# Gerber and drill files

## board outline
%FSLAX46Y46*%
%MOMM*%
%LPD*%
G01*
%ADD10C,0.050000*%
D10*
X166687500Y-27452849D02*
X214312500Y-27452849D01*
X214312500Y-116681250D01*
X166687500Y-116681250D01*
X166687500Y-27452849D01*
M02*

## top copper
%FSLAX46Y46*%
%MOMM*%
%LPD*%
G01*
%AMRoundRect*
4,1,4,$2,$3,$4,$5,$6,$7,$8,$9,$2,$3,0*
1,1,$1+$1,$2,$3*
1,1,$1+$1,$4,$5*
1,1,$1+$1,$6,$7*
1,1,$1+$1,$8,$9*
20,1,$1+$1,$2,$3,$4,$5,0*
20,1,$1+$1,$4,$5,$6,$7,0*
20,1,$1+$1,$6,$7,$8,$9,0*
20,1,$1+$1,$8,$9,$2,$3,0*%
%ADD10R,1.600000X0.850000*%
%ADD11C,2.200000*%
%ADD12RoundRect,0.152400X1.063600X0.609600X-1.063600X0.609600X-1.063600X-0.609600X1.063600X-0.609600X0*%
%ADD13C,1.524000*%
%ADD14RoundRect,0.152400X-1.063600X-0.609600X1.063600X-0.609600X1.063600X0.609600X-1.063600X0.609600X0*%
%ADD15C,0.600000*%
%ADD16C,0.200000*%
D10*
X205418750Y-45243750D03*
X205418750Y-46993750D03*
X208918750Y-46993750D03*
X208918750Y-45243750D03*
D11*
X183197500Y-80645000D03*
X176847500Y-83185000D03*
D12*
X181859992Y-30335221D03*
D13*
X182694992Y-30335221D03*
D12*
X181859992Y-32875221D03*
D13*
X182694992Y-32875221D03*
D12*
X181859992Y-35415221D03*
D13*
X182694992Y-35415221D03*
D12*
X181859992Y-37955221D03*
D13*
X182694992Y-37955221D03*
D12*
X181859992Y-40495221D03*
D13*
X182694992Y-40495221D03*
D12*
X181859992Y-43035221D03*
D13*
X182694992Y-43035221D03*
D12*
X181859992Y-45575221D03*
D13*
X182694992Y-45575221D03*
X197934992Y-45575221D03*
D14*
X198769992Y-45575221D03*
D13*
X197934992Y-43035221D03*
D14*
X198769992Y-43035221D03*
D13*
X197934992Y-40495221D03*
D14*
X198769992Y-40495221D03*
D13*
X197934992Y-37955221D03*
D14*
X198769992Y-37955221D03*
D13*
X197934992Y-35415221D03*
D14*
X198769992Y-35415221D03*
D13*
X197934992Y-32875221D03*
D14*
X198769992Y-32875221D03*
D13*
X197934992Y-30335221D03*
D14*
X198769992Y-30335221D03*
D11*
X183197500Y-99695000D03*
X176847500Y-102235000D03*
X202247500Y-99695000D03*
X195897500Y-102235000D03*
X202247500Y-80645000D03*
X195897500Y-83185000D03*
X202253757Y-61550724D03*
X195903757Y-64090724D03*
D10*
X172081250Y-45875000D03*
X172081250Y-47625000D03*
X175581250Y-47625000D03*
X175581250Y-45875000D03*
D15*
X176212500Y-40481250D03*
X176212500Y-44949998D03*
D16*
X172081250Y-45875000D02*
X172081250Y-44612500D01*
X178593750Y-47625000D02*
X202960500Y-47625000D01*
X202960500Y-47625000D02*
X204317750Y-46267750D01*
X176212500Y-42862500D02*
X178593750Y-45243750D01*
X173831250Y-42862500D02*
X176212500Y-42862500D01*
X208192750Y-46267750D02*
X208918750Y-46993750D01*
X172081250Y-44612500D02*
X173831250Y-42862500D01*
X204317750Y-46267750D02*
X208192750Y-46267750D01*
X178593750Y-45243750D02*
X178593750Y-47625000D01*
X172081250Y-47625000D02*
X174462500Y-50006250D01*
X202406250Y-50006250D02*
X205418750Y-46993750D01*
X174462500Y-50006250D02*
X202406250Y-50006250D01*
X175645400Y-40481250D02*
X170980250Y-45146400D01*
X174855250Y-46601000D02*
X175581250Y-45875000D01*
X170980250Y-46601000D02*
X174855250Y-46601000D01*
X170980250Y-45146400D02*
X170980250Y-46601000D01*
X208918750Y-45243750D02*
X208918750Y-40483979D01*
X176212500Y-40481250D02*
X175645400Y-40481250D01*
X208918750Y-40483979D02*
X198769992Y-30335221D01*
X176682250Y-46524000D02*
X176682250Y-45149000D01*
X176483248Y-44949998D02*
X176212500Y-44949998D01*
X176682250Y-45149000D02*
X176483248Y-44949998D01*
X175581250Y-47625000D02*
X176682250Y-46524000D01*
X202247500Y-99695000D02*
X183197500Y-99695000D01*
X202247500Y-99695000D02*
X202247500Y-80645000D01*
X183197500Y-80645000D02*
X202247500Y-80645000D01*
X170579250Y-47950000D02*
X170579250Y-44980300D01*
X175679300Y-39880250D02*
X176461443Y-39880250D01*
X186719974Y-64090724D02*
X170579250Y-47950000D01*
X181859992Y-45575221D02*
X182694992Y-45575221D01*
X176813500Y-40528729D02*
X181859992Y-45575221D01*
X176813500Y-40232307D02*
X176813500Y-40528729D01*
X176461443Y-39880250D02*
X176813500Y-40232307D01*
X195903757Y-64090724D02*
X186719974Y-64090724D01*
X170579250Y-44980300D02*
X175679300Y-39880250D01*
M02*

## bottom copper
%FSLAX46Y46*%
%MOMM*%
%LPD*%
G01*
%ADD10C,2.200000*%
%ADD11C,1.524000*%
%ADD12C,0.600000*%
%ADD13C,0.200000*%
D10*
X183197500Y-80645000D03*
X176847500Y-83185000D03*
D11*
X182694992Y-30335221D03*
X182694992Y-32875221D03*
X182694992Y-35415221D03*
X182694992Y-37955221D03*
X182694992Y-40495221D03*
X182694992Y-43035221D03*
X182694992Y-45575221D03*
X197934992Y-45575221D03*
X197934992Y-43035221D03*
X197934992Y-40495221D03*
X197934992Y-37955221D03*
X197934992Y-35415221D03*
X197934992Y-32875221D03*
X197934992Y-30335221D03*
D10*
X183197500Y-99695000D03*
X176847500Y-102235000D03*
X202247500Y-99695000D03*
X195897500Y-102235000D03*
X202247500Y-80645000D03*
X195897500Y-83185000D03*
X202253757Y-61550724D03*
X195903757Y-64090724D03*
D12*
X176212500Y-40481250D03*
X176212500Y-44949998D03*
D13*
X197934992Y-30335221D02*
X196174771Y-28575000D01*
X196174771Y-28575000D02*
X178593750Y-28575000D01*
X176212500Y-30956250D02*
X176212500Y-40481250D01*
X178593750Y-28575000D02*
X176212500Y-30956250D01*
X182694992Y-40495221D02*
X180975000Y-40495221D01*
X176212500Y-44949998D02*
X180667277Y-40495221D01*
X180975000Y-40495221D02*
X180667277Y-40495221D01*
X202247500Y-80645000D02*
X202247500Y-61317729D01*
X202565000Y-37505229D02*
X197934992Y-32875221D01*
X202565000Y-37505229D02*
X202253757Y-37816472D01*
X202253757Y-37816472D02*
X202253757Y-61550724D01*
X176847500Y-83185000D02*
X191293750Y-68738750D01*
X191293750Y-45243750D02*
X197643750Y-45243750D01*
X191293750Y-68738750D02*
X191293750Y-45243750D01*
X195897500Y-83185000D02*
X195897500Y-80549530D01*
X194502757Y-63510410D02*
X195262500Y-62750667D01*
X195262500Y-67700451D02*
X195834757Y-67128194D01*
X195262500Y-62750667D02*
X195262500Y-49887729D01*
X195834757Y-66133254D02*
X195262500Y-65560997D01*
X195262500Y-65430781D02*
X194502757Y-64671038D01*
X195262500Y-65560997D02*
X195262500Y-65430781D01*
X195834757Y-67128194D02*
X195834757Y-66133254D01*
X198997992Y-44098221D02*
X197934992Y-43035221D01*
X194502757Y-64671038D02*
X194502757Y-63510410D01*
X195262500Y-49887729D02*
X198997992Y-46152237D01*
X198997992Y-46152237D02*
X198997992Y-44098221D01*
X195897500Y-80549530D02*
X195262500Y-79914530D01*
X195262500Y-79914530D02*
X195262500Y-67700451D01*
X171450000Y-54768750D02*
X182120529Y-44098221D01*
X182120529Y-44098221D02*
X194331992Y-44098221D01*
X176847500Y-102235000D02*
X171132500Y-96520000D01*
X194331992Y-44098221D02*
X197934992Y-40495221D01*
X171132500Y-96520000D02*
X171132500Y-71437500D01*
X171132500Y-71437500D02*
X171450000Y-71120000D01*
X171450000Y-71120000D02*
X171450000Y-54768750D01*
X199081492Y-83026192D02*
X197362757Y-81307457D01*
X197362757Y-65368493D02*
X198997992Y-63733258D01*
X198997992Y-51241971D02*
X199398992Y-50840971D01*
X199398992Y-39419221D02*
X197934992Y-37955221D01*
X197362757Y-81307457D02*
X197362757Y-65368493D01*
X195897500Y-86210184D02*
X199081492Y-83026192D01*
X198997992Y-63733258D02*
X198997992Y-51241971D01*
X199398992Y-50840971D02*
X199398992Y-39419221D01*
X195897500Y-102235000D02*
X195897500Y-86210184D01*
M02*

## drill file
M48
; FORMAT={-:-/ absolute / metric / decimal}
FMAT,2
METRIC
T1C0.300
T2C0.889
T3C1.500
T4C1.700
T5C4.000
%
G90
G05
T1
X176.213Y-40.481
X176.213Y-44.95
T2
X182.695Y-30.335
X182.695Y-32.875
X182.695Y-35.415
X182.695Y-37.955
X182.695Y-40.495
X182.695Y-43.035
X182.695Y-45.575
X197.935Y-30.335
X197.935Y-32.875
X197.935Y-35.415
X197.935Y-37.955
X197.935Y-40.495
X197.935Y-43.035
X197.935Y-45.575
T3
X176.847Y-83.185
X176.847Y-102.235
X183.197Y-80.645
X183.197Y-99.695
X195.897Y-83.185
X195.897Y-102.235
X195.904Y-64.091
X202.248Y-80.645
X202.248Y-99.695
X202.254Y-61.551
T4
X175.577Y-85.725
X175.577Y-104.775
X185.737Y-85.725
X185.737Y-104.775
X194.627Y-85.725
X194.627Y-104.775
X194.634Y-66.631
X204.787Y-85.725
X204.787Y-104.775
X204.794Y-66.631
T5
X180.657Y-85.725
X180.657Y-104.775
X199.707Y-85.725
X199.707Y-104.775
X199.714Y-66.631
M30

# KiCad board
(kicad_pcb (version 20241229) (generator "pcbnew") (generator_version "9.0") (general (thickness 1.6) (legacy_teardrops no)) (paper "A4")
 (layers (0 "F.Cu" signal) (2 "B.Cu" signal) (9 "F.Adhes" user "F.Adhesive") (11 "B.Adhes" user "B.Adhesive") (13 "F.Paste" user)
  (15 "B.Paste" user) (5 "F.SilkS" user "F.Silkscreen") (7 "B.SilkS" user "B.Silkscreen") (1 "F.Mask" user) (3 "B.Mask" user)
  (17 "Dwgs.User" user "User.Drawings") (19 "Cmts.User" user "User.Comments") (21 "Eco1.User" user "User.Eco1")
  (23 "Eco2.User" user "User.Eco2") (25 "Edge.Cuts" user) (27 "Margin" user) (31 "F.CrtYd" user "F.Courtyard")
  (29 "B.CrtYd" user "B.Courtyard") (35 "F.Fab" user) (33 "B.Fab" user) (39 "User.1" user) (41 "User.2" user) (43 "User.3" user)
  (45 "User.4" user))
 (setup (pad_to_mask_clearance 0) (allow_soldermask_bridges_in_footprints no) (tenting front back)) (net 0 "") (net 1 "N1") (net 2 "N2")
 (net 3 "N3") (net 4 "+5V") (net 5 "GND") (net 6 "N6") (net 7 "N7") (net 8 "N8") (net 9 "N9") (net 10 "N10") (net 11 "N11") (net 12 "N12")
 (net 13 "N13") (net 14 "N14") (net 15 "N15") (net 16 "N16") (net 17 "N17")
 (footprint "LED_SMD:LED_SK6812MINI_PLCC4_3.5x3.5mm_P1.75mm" (layer "F.Cu") (at 207.16875 46.11875)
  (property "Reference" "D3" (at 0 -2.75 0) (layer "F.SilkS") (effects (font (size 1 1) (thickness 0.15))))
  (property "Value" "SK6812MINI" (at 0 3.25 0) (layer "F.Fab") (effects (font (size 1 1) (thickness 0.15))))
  (pad "1" smd rect (at -1.75 -0.875) (size 1.6 0.85) (layers "F.Cu" "F.Mask" "F.Paste") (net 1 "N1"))
  (pad "2" smd rect (at -1.75 0.875) (size 1.6 0.85) (layers "F.Cu" "F.Mask" "F.Paste") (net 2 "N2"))
  (pad "3" smd rect (at 1.75 0.875) (size 1.6 0.85) (layers "F.Cu" "F.Mask" "F.Paste") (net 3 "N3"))
  (pad "4" smd rect (at 1.75 -0.875) (size 1.6 0.85) (layers "F.Cu" "F.Mask" "F.Paste") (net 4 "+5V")))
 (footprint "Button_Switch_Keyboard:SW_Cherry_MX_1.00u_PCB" (layer "F.Cu") (at 183.1975 80.645)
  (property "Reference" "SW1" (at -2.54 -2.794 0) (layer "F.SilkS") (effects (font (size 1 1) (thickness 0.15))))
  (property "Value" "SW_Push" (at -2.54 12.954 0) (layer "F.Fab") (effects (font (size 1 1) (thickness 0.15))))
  (pad "" np_thru_hole circle (at -7.62 5.08) (size 1.7 1.7) (drill 1.7) (layers "*.Cu" "*.Mask"))
  (pad "" np_thru_hole circle (at -2.54 5.08) (size 4 4) (drill 4) (layers "*.Cu" "*.Mask"))
  (pad "" np_thru_hole circle (at 2.54 5.08) (size 1.7 1.7) (drill 1.7) (layers "*.Cu" "*.Mask"))
  (pad "1" thru_hole circle (at 0 0) (size 2.2 2.2) (drill 1.5) (layers "*.Cu" "*.Mask") (remove_unused_layers no) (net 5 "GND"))
  (pad "2" thru_hole circle (at -6.35 2.54) (size 2.2 2.2) (drill 1.5) (layers "*.Cu" "*.Mask") (remove_unused_layers no) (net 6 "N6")))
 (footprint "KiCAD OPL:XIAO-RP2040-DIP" (layer "F.Cu") (at 190.314992 37.955221)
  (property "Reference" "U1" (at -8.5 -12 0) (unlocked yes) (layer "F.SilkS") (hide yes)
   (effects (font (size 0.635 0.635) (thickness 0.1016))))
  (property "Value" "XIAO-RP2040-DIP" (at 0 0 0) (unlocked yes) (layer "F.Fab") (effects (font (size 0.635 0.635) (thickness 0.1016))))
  (pad "1" smd roundrect (at -8.455 -7.62 180) (size 2.432 1.524) (layers "F.Cu" "F.Mask") (roundrect_rratio 0.1) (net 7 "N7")
   (thermal_bridge_angle 45))
  (pad "1" thru_hole circle (at -7.62 -7.62 180) (size 1.524 1.524) (drill 0.889) (layers "*.Cu" "*.Mask") (remove_unused_layers no)
   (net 7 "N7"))
  (pad "2" smd roundrect (at -8.455 -5.08 180) (size 2.432 1.524) (layers "F.Cu" "F.Mask") (roundrect_rratio 0.1) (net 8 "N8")
   (thermal_bridge_angle 45))
  (pad "2" thru_hole circle (at -7.62 -5.08 180) (size 1.524 1.524) (drill 0.889) (layers "*.Cu" "*.Mask") (remove_unused_layers no)
   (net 8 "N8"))
  (pad "3" smd roundrect (at -8.455 -2.54 180) (size 2.432 1.524) (layers "F.Cu" "F.Mask") (roundrect_rratio 0.1) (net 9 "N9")
   (thermal_bridge_angle 45))
  (pad "3" thru_hole circle (at -7.62 -2.54 180) (size 1.524 1.524) (drill 0.889) (layers "*.Cu" "*.Mask") (remove_unused_layers no)
   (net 9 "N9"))
  (pad "4" smd roundrect (at -8.455 0 180) (size 2.432 1.524) (layers "F.Cu" "F.Mask") (roundrect_rratio 0.1) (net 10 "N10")
   (thermal_bridge_angle 45))
  (pad "4" thru_hole circle (at -7.62 0 180) (size 1.524 1.524) (drill 0.889) (layers "*.Cu" "*.Mask") (remove_unused_layers no)
   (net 10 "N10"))
  (pad "5" smd roundrect (at -8.455 2.54 180) (size 2.432 1.524) (layers "F.Cu" "F.Mask") (roundrect_rratio 0.1) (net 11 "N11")
   (thermal_bridge_angle 45))
  (pad "5" thru_hole circle (at -7.62 2.54 180) (size 1.524 1.524) (drill 0.889) (layers "*.Cu" "*.Mask") (remove_unused_layers no)
   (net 11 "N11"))
  (pad "6" smd roundrect (at -8.455 5.08 180) (size 2.432 1.524) (layers "F.Cu" "F.Mask") (roundrect_rratio 0.1) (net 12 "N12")
   (thermal_bridge_angle 45))
  (pad "6" thru_hole circle (at -7.62 5.08 180) (size 1.524 1.524) (drill 0.889) (layers "*.Cu" "*.Mask") (remove_unused_layers no)
   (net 12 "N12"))
  (pad "7" smd roundrect (at -8.455 7.62 180) (size 2.432 1.524) (layers "F.Cu" "F.Mask") (roundrect_rratio 0.1) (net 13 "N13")
   (thermal_bridge_angle 45))
  (pad "7" thru_hole circle (at -7.62 7.62 180) (size 1.524 1.524) (drill 0.889) (layers "*.Cu" "*.Mask") (remove_unused_layers no)
   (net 13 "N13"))
  (pad "8" thru_hole circle (at 7.62 7.62) (size 1.524 1.524) (drill 0.889) (layers "*.Cu" "*.Mask") (remove_unused_layers no) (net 6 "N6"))
  (pad "8" smd roundrect (at 8.455 7.62) (size 2.432 1.524) (layers "F.Cu" "F.Mask") (roundrect_rratio 0.1) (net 6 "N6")
   (thermal_bridge_angle 45))
  (pad "9" thru_hole circle (at 7.62 5.08) (size 1.524 1.524) (drill 0.889) (layers "*.Cu" "*.Mask") (remove_unused_layers no)
   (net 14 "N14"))
  (pad "9" smd roundrect (at 8.455 5.08) (size 2.432 1.524) (layers "F.Cu" "F.Mask") (roundrect_rratio 0.1) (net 14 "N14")
   (thermal_bridge_angle 45))
  (pad "10" thru_hole circle (at 7.62 2.54) (size 1.524 1.524) (drill 0.889) (layers "*.Cu" "*.Mask") (remove_unused_layers no)
   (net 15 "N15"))
  (pad "10" smd roundrect (at 8.455 2.54) (size 2.432 1.524) (layers "F.Cu" "F.Mask") (roundrect_rratio 0.1) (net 15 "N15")
   (thermal_bridge_angle 45))
  (pad "11" thru_hole circle (at 7.62 0) (size 1.524 1.524) (drill 0.889) (layers "*.Cu" "*.Mask") (remove_unused_layers no) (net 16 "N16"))
  (pad "11" smd roundrect (at 8.455 0) (size 2.432 1.524) (layers "F.Cu" "F.Mask") (roundrect_rratio 0.1) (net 16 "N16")
   (thermal_bridge_angle 45))
  (pad "12" thru_hole circle (at 7.62 -2.54) (size 1.524 1.524) (drill 0.889) (layers "*.Cu" "*.Mask") (remove_unused_layers no)
   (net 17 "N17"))
  (pad "12" smd roundrect (at 8.455 -2.54) (size 2.432 1.524) (layers "F.Cu" "F.Mask") (roundrect_rratio 0.1) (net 17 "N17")
   (thermal_bridge_angle 45))
  (pad "13" thru_hole circle (at 7.62 -5.08) (size 1.524 1.524) (drill 0.889) (layers "*.Cu" "*.Mask") (remove_unused_layers no)
   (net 5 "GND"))
  (pad "13" smd roundrect (at 8.455 -5.08) (size 2.432 1.524) (layers "F.Cu" "F.Mask") (roundrect_rratio 0.1) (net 5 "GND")
   (thermal_bridge_angle 45))
  (pad "14" thru_hole circle (at 7.62 -7.62) (size 1.524 1.524) (drill 0.889) (layers "*.Cu" "*.Mask") (remove_unused_layers no)
   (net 4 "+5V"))
  (pad "14" smd roundrect (at 8.455 -7.62) (size 2.432 1.524) (layers "F.Cu" "F.Mask") (roundrect_rratio 0.1) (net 4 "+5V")
   (thermal_bridge_angle 45)))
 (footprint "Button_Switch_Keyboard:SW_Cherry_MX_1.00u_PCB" (layer "F.Cu") (at 183.1975 99.695)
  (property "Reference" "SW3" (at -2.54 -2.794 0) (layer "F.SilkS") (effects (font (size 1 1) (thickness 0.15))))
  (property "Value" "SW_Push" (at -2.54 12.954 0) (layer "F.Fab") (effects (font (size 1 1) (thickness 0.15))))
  (pad "" np_thru_hole circle (at -7.62 5.08) (size 1.7 1.7) (drill 1.7) (layers "*.Cu" "*.Mask"))
  (pad "" np_thru_hole circle (at -2.54 5.08) (size 4 4) (drill 4) (layers "*.Cu" "*.Mask"))
  (pad "" np_thru_hole circle (at 2.54 5.08) (size 1.7 1.7) (drill 1.7) (layers "*.Cu" "*.Mask"))
  (pad "1" thru_hole circle (at 0 0) (size 2.2 2.2) (drill 1.5) (layers "*.Cu" "*.Mask") (remove_unused_layers no) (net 5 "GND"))
  (pad "2" thru_hole circle (at -6.35 2.54) (size 2.2 2.2) (drill 1.5) (layers "*.Cu" "*.Mask") (remove_unused_layers no) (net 15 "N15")))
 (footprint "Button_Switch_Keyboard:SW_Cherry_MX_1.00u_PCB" (layer "F.Cu") (at 202.2475 99.695)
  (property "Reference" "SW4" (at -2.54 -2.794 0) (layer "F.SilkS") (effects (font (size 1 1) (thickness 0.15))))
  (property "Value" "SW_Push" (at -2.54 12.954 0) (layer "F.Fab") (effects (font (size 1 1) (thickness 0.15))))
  (pad "" np_thru_hole circle (at -7.62 5.08) (size 1.7 1.7) (drill 1.7) (layers "*.Cu" "*.Mask"))
  (pad "" np_thru_hole circle (at -2.54 5.08) (size 4 4) (drill 4) (layers "*.Cu" "*.Mask"))
  (pad "" np_thru_hole circle (at 2.54 5.08) (size 1.7 1.7) (drill 1.7) (layers "*.Cu" "*.Mask"))
  (pad "1" thru_hole circle (at 0 0) (size 2.2 2.2) (drill 1.5) (layers "*.Cu" "*.Mask") (remove_unused_layers no) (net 5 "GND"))
  (pad "2" thru_hole circle (at -6.35 2.54) (size 2.2 2.2) (drill 1.5) (layers "*.Cu" "*.Mask") (remove_unused_layers no) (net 16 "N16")))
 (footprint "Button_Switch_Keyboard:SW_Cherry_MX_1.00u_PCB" (layer "F.Cu") (at 202.2475 80.645)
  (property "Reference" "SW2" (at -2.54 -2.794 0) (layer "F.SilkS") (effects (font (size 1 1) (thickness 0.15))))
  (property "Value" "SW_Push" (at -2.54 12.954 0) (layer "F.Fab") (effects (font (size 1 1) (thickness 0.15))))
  (pad "" np_thru_hole circle (at -7.62 5.08) (size 1.7 1.7) (drill 1.7) (layers "*.Cu" "*.Mask"))
  (pad "" np_thru_hole circle (at -2.54 5.08) (size 4 4) (drill 4) (layers "*.Cu" "*.Mask"))
  (pad "" np_thru_hole circle (at 2.54 5.08) (size 1.7 1.7) (drill 1.7) (layers "*.Cu" "*.Mask"))
  (pad "1" thru_hole circle (at 0 0) (size 2.2 2.2) (drill 1.5) (layers "*.Cu" "*.Mask") (remove_unused_layers no) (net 5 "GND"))
  (pad "2" thru_hole circle (at -6.35 2.54) (size 2.2 2.2) (drill 1.5) (layers "*.Cu" "*.Mask") (remove_unused_layers no) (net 14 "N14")))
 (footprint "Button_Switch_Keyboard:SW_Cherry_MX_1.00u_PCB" (layer "F.Cu") (at 202.253757 61.550724)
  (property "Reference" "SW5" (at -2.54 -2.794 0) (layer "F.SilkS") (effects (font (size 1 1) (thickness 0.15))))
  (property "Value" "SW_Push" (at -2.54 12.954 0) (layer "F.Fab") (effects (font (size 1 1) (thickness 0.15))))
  (pad "" np_thru_hole circle (at -7.62 5.08) (size 1.7 1.7) (drill 1.7) (layers "*.Cu" "*.Mask"))
  (pad "" np_thru_hole circle (at -2.54 5.08) (size 4 4) (drill 4) (layers "*.Cu" "*.Mask"))
  (pad "" np_thru_hole circle (at 2.54 5.08) (size 1.7 1.7) (drill 1.7) (layers "*.Cu" "*.Mask"))
  (pad "1" thru_hole circle (at 0 0) (size 2.2 2.2) (drill 1.5) (layers "*.Cu" "*.Mask") (remove_unused_layers no) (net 5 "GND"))
  (pad "2" thru_hole circle (at -6.35 2.54) (size 2.2 2.2) (drill 1.5) (layers "*.Cu" "*.Mask") (remove_unused_layers no) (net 13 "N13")))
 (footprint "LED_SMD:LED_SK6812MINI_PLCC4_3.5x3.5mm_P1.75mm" (layer "F.Cu") (at 173.83125 46.75)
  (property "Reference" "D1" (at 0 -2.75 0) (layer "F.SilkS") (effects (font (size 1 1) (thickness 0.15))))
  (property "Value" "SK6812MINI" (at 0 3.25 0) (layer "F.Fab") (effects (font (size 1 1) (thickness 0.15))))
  (pad "1" smd rect (at -1.75 -0.875) (size 1.6 0.85) (layers "F.Cu" "F.Mask" "F.Paste") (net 3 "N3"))
  (pad "2" smd rect (at -1.75 0.875) (size 1.6 0.85) (layers "F.Cu" "F.Mask" "F.Paste") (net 2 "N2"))
  (pad "3" smd rect (at 1.75 0.875) (size 1.6 0.85) (layers "F.Cu" "F.Mask" "F.Paste") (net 11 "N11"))
  (pad "4" smd rect (at 1.75 -0.875) (size 1.6 0.85) (layers "F.Cu" "F.Mask" "F.Paste") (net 4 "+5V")))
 (gr_rect (start 166.6875 27.452849) (end 214.3125 116.68125) (stroke (width 0.05) (type default)) (fill no) (layer "Edge.Cuts"))
 (segment (start 172.08125 45.875) (end 172.08125 44.6125) (width 0.2) (layer "F.Cu") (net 3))
 (segment (start 178.59375 47.625) (end 202.9605 47.625) (width 0.2) (layer "F.Cu") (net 3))
 (segment (start 202.9605 47.625) (end 204.31775 46.26775) (width 0.2) (layer "F.Cu") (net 3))
 (segment (start 176.2125 42.8625) (end 178.59375 45.24375) (width 0.2) (layer "F.Cu") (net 3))
 (segment (start 173.83125 42.8625) (end 176.2125 42.8625) (width 0.2) (layer "F.Cu") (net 3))
 (segment (start 208.19275 46.26775) (end 208.91875 46.99375) (width 0.2) (layer "F.Cu") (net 3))
 (segment (start 172.08125 44.6125) (end 173.83125 42.8625) (width 0.2) (layer "F.Cu") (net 3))
 (segment (start 204.31775 46.26775) (end 208.19275 46.26775) (width 0.2) (layer "F.Cu") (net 3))
 (segment (start 178.59375 45.24375) (end 178.59375 47.625) (width 0.2) (layer "F.Cu") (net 3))
 (segment (start 172.08125 47.625) (end 174.4625 50.00625) (width 0.2) (layer "F.Cu") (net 2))
 (segment (start 202.40625 50.00625) (end 205.41875 46.99375) (width 0.2) (layer "F.Cu") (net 2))
 (segment (start 174.4625 50.00625) (end 202.40625 50.00625) (width 0.2) (layer "F.Cu") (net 2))
 (segment (start 175.6454 40.48125) (end 170.98025 45.1464) (width 0.2) (layer "F.Cu") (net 4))
 (segment (start 174.85525 46.601) (end 175.58125 45.875) (width 0.2) (layer "F.Cu") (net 4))
 (segment (start 170.98025 46.601) (end 174.85525 46.601) (width 0.2) (layer "F.Cu") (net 4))
 (segment (start 170.98025 45.1464) (end 170.98025 46.601) (width 0.2) (layer "F.Cu") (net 4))
 (segment (start 208.91875 45.24375) (end 208.91875 40.483979) (width 0.2) (layer "F.Cu") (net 4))
 (segment (start 176.2125 40.48125) (end 175.6454 40.48125) (width 0.2) (layer "F.Cu") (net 4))
 (segment (start 208.91875 40.483979) (end 198.769992 30.335221) (width 0.2) (layer "F.Cu") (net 4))
 (via (at 176.2125 40.48125) (size 0.6) (drill 0.3) (layers "F.Cu" "B.Cu") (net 4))
 (segment (start 197.934992 30.335221) (end 196.174771 28.575) (width 0.2) (layer "B.Cu") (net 4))
 (segment (start 196.174771 28.575) (end 178.59375 28.575) (width 0.2) (layer "B.Cu") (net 4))
 (segment (start 176.2125 30.95625) (end 176.2125 40.48125) (width 0.2) (layer "B.Cu") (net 4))
 (segment (start 178.59375 28.575) (end 176.2125 30.95625) (width 0.2) (layer "B.Cu") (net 4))
 (segment (start 176.68225 46.524) (end 176.68225 45.149) (width 0.2) (layer "F.Cu") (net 11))
 (segment (start 176.483248 44.949998) (end 176.2125 44.949998) (width 0.2) (layer "F.Cu") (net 11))
 (segment (start 176.68225 45.149) (end 176.483248 44.949998) (width 0.2) (layer "F.Cu") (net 11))
 (segment (start 175.58125 47.625) (end 176.68225 46.524) (width 0.2) (layer "F.Cu") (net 11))
 (via (at 176.2125 44.949998) (size 0.6) (drill 0.3) (layers "F.Cu" "B.Cu") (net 11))
 (segment (start 182.694992 40.495221) (end 180.975 40.495221) (width 0.2) (layer "B.Cu") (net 11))
 (segment (start 176.2125 44.949998) (end 180.667277 40.495221) (width 0.2) (layer "B.Cu") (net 11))
 (segment (start 180.975 40.495221) (end 180.667277 40.495221) (width 0.2) (layer "B.Cu") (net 11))
 (segment (start 202.2475 99.695) (end 183.1975 99.695) (width 0.2) (layer "F.Cu") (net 5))
 (segment (start 202.2475 99.695) (end 202.2475 80.645) (width 0.2) (layer "F.Cu") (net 5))
 (segment (start 183.1975 80.645) (end 202.2475 80.645) (width 0.2) (layer "F.Cu") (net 5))
 (segment (start 202.2475 80.645) (end 202.2475 61.317729) (width 0.2) (layer "B.Cu") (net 5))
 (segment (start 202.565 37.505229) (end 197.934992 32.875221) (width 0.2) (layer "B.Cu") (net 5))
 (segment (start 202.565 37.505229) (end 202.253757 37.816472) (width 0.2) (layer "B.Cu") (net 5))
 (segment (start 202.253757 37.816472) (end 202.253757 61.550724) (width 0.2) (layer "B.Cu") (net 5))
 (segment (start 176.8475 83.185) (end 191.29375 68.73875) (width 0.2) (layer "B.Cu") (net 6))
 (segment (start 191.29375 45.24375) (end 197.64375 45.24375) (width 0.2) (layer "B.Cu") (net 6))
 (segment (start 191.29375 68.73875) (end 191.29375 45.24375) (width 0.2) (layer "B.Cu") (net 6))
 (segment (start 195.8975 83.185) (end 195.8975 80.54953) (width 0.2) (layer "B.Cu") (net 14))
 (segment (start 194.502757 63.51041) (end 195.2625 62.750667) (width 0.2) (layer "B.Cu") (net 14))
 (segment (start 195.2625 67.700451) (end 195.834757 67.128194) (width 0.2) (layer "B.Cu") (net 14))
 (segment (start 195.2625 62.750667) (end 195.2625 49.887729) (width 0.2) (layer "B.Cu") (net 14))
 (segment (start 195.834757 66.133254) (end 195.2625 65.560997) (width 0.2) (layer "B.Cu") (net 14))
 (segment (start 195.2625 65.430781) (end 194.502757 64.671038) (width 0.2) (layer "B.Cu") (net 14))
 (segment (start 195.2625 65.560997) (end 195.2625 65.430781) (width 0.2) (layer "B.Cu") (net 14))
 (segment (start 195.834757 67.128194) (end 195.834757 66.133254) (width 0.2) (layer "B.Cu") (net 14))
 (segment (start 198.997992 44.098221) (end 197.934992 43.035221) (width 0.2) (layer "B.Cu") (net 14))
 (segment (start 194.502757 64.671038) (end 194.502757 63.51041) (width 0.2) (layer "B.Cu") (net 14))
 (segment (start 195.2625 49.887729) (end 198.997992 46.152237) (width 0.2) (layer "B.Cu") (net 14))
 (segment (start 198.997992 46.152237) (end 198.997992 44.098221) (width 0.2) (layer "B.Cu") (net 14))
 (segment (start 195.8975 80.54953) (end 195.2625 79.91453) (width 0.2) (layer "B.Cu") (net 14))
 (segment (start 195.2625 79.91453) (end 195.2625 67.700451) (width 0.2) (layer "B.Cu") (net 14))
 (segment (start 171.45 54.76875) (end 182.120529 44.098221) (width 0.2) (layer "B.Cu") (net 15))
 (segment (start 182.120529 44.098221) (end 194.331992 44.098221) (width 0.2) (layer "B.Cu") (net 15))
 (segment (start 176.8475 102.235) (end 171.1325 96.52) (width 0.2) (layer "B.Cu") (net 15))
 (segment (start 194.331992 44.098221) (end 197.934992 40.495221) (width 0.2) (layer "B.Cu") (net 15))
 (segment (start 171.1325 96.52) (end 171.1325 71.4375) (width 0.2) (layer "B.Cu") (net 15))
 (segment (start 171.1325 71.4375) (end 171.45 71.12) (width 0.2) (layer "B.Cu") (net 15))
 (segment (start 171.45 71.12) (end 171.45 54.76875) (width 0.2) (layer "B.Cu") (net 15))
 (segment (start 199.081492 83.026192) (end 197.362757 81.307457) (width 0.2) (layer "B.Cu") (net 16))
 (segment (start 197.362757 65.368493) (end 198.997992 63.733258) (width 0.2) (layer "B.Cu") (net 16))
 (segment (start 198.997992 51.241971) (end 199.398992 50.840971) (width 0.2) (layer "B.Cu") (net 16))
 (segment (start 199.398992 39.419221) (end 197.934992 37.955221) (width 0.2) (layer "B.Cu") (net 16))
 (segment (start 197.362757 81.307457) (end 197.362757 65.368493) (width 0.2) (layer "B.Cu") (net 16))
 (segment (start 195.8975 86.210184) (end 199.081492 83.026192) (width 0.2) (layer "B.Cu") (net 16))
 (segment (start 198.997992 63.733258) (end 198.997992 51.241971) (width 0.2) (layer "B.Cu") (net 16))
 (segment (start 199.398992 50.840971) (end 199.398992 39.419221) (width 0.2) (layer "B.Cu") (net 16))
 (segment (start 195.8975 102.235) (end 195.8975 86.210184) (width 0.2) (layer "B.Cu") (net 16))
 (segment (start 170.57925 47.95) (end 170.57925 44.9803) (width 0.2) (layer "F.Cu") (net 13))
 (segment (start 175.6793 39.88025) (end 176.461443 39.88025) (width 0.2) (layer "F.Cu") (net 13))
 (segment (start 186.719974 64.090724) (end 170.57925 47.95) (width 0.2) (layer "F.Cu") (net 13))
 (segment (start 181.859992 45.575221) (end 182.694992 45.575221) (width 0.2) (layer "F.Cu") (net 13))
 (segment (start 176.8135 40.528729) (end 181.859992 45.575221) (width 0.2) (layer "F.Cu") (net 13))
 (segment (start 176.8135 40.232307) (end 176.8135 40.528729) (width 0.2) (layer "F.Cu") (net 13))
 (segment (start 176.461443 39.88025) (end 176.8135 40.232307) (width 0.2) (layer "F.Cu") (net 13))
 (segment (start 195.903757 64.090724) (end 186.719974 64.090724) (width 0.2) (layer "F.Cu") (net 13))
 (segment (start 170.57925 44.9803) (end 175.6793 39.88025) (width 0.2) (layer "F.Cu") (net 13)))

